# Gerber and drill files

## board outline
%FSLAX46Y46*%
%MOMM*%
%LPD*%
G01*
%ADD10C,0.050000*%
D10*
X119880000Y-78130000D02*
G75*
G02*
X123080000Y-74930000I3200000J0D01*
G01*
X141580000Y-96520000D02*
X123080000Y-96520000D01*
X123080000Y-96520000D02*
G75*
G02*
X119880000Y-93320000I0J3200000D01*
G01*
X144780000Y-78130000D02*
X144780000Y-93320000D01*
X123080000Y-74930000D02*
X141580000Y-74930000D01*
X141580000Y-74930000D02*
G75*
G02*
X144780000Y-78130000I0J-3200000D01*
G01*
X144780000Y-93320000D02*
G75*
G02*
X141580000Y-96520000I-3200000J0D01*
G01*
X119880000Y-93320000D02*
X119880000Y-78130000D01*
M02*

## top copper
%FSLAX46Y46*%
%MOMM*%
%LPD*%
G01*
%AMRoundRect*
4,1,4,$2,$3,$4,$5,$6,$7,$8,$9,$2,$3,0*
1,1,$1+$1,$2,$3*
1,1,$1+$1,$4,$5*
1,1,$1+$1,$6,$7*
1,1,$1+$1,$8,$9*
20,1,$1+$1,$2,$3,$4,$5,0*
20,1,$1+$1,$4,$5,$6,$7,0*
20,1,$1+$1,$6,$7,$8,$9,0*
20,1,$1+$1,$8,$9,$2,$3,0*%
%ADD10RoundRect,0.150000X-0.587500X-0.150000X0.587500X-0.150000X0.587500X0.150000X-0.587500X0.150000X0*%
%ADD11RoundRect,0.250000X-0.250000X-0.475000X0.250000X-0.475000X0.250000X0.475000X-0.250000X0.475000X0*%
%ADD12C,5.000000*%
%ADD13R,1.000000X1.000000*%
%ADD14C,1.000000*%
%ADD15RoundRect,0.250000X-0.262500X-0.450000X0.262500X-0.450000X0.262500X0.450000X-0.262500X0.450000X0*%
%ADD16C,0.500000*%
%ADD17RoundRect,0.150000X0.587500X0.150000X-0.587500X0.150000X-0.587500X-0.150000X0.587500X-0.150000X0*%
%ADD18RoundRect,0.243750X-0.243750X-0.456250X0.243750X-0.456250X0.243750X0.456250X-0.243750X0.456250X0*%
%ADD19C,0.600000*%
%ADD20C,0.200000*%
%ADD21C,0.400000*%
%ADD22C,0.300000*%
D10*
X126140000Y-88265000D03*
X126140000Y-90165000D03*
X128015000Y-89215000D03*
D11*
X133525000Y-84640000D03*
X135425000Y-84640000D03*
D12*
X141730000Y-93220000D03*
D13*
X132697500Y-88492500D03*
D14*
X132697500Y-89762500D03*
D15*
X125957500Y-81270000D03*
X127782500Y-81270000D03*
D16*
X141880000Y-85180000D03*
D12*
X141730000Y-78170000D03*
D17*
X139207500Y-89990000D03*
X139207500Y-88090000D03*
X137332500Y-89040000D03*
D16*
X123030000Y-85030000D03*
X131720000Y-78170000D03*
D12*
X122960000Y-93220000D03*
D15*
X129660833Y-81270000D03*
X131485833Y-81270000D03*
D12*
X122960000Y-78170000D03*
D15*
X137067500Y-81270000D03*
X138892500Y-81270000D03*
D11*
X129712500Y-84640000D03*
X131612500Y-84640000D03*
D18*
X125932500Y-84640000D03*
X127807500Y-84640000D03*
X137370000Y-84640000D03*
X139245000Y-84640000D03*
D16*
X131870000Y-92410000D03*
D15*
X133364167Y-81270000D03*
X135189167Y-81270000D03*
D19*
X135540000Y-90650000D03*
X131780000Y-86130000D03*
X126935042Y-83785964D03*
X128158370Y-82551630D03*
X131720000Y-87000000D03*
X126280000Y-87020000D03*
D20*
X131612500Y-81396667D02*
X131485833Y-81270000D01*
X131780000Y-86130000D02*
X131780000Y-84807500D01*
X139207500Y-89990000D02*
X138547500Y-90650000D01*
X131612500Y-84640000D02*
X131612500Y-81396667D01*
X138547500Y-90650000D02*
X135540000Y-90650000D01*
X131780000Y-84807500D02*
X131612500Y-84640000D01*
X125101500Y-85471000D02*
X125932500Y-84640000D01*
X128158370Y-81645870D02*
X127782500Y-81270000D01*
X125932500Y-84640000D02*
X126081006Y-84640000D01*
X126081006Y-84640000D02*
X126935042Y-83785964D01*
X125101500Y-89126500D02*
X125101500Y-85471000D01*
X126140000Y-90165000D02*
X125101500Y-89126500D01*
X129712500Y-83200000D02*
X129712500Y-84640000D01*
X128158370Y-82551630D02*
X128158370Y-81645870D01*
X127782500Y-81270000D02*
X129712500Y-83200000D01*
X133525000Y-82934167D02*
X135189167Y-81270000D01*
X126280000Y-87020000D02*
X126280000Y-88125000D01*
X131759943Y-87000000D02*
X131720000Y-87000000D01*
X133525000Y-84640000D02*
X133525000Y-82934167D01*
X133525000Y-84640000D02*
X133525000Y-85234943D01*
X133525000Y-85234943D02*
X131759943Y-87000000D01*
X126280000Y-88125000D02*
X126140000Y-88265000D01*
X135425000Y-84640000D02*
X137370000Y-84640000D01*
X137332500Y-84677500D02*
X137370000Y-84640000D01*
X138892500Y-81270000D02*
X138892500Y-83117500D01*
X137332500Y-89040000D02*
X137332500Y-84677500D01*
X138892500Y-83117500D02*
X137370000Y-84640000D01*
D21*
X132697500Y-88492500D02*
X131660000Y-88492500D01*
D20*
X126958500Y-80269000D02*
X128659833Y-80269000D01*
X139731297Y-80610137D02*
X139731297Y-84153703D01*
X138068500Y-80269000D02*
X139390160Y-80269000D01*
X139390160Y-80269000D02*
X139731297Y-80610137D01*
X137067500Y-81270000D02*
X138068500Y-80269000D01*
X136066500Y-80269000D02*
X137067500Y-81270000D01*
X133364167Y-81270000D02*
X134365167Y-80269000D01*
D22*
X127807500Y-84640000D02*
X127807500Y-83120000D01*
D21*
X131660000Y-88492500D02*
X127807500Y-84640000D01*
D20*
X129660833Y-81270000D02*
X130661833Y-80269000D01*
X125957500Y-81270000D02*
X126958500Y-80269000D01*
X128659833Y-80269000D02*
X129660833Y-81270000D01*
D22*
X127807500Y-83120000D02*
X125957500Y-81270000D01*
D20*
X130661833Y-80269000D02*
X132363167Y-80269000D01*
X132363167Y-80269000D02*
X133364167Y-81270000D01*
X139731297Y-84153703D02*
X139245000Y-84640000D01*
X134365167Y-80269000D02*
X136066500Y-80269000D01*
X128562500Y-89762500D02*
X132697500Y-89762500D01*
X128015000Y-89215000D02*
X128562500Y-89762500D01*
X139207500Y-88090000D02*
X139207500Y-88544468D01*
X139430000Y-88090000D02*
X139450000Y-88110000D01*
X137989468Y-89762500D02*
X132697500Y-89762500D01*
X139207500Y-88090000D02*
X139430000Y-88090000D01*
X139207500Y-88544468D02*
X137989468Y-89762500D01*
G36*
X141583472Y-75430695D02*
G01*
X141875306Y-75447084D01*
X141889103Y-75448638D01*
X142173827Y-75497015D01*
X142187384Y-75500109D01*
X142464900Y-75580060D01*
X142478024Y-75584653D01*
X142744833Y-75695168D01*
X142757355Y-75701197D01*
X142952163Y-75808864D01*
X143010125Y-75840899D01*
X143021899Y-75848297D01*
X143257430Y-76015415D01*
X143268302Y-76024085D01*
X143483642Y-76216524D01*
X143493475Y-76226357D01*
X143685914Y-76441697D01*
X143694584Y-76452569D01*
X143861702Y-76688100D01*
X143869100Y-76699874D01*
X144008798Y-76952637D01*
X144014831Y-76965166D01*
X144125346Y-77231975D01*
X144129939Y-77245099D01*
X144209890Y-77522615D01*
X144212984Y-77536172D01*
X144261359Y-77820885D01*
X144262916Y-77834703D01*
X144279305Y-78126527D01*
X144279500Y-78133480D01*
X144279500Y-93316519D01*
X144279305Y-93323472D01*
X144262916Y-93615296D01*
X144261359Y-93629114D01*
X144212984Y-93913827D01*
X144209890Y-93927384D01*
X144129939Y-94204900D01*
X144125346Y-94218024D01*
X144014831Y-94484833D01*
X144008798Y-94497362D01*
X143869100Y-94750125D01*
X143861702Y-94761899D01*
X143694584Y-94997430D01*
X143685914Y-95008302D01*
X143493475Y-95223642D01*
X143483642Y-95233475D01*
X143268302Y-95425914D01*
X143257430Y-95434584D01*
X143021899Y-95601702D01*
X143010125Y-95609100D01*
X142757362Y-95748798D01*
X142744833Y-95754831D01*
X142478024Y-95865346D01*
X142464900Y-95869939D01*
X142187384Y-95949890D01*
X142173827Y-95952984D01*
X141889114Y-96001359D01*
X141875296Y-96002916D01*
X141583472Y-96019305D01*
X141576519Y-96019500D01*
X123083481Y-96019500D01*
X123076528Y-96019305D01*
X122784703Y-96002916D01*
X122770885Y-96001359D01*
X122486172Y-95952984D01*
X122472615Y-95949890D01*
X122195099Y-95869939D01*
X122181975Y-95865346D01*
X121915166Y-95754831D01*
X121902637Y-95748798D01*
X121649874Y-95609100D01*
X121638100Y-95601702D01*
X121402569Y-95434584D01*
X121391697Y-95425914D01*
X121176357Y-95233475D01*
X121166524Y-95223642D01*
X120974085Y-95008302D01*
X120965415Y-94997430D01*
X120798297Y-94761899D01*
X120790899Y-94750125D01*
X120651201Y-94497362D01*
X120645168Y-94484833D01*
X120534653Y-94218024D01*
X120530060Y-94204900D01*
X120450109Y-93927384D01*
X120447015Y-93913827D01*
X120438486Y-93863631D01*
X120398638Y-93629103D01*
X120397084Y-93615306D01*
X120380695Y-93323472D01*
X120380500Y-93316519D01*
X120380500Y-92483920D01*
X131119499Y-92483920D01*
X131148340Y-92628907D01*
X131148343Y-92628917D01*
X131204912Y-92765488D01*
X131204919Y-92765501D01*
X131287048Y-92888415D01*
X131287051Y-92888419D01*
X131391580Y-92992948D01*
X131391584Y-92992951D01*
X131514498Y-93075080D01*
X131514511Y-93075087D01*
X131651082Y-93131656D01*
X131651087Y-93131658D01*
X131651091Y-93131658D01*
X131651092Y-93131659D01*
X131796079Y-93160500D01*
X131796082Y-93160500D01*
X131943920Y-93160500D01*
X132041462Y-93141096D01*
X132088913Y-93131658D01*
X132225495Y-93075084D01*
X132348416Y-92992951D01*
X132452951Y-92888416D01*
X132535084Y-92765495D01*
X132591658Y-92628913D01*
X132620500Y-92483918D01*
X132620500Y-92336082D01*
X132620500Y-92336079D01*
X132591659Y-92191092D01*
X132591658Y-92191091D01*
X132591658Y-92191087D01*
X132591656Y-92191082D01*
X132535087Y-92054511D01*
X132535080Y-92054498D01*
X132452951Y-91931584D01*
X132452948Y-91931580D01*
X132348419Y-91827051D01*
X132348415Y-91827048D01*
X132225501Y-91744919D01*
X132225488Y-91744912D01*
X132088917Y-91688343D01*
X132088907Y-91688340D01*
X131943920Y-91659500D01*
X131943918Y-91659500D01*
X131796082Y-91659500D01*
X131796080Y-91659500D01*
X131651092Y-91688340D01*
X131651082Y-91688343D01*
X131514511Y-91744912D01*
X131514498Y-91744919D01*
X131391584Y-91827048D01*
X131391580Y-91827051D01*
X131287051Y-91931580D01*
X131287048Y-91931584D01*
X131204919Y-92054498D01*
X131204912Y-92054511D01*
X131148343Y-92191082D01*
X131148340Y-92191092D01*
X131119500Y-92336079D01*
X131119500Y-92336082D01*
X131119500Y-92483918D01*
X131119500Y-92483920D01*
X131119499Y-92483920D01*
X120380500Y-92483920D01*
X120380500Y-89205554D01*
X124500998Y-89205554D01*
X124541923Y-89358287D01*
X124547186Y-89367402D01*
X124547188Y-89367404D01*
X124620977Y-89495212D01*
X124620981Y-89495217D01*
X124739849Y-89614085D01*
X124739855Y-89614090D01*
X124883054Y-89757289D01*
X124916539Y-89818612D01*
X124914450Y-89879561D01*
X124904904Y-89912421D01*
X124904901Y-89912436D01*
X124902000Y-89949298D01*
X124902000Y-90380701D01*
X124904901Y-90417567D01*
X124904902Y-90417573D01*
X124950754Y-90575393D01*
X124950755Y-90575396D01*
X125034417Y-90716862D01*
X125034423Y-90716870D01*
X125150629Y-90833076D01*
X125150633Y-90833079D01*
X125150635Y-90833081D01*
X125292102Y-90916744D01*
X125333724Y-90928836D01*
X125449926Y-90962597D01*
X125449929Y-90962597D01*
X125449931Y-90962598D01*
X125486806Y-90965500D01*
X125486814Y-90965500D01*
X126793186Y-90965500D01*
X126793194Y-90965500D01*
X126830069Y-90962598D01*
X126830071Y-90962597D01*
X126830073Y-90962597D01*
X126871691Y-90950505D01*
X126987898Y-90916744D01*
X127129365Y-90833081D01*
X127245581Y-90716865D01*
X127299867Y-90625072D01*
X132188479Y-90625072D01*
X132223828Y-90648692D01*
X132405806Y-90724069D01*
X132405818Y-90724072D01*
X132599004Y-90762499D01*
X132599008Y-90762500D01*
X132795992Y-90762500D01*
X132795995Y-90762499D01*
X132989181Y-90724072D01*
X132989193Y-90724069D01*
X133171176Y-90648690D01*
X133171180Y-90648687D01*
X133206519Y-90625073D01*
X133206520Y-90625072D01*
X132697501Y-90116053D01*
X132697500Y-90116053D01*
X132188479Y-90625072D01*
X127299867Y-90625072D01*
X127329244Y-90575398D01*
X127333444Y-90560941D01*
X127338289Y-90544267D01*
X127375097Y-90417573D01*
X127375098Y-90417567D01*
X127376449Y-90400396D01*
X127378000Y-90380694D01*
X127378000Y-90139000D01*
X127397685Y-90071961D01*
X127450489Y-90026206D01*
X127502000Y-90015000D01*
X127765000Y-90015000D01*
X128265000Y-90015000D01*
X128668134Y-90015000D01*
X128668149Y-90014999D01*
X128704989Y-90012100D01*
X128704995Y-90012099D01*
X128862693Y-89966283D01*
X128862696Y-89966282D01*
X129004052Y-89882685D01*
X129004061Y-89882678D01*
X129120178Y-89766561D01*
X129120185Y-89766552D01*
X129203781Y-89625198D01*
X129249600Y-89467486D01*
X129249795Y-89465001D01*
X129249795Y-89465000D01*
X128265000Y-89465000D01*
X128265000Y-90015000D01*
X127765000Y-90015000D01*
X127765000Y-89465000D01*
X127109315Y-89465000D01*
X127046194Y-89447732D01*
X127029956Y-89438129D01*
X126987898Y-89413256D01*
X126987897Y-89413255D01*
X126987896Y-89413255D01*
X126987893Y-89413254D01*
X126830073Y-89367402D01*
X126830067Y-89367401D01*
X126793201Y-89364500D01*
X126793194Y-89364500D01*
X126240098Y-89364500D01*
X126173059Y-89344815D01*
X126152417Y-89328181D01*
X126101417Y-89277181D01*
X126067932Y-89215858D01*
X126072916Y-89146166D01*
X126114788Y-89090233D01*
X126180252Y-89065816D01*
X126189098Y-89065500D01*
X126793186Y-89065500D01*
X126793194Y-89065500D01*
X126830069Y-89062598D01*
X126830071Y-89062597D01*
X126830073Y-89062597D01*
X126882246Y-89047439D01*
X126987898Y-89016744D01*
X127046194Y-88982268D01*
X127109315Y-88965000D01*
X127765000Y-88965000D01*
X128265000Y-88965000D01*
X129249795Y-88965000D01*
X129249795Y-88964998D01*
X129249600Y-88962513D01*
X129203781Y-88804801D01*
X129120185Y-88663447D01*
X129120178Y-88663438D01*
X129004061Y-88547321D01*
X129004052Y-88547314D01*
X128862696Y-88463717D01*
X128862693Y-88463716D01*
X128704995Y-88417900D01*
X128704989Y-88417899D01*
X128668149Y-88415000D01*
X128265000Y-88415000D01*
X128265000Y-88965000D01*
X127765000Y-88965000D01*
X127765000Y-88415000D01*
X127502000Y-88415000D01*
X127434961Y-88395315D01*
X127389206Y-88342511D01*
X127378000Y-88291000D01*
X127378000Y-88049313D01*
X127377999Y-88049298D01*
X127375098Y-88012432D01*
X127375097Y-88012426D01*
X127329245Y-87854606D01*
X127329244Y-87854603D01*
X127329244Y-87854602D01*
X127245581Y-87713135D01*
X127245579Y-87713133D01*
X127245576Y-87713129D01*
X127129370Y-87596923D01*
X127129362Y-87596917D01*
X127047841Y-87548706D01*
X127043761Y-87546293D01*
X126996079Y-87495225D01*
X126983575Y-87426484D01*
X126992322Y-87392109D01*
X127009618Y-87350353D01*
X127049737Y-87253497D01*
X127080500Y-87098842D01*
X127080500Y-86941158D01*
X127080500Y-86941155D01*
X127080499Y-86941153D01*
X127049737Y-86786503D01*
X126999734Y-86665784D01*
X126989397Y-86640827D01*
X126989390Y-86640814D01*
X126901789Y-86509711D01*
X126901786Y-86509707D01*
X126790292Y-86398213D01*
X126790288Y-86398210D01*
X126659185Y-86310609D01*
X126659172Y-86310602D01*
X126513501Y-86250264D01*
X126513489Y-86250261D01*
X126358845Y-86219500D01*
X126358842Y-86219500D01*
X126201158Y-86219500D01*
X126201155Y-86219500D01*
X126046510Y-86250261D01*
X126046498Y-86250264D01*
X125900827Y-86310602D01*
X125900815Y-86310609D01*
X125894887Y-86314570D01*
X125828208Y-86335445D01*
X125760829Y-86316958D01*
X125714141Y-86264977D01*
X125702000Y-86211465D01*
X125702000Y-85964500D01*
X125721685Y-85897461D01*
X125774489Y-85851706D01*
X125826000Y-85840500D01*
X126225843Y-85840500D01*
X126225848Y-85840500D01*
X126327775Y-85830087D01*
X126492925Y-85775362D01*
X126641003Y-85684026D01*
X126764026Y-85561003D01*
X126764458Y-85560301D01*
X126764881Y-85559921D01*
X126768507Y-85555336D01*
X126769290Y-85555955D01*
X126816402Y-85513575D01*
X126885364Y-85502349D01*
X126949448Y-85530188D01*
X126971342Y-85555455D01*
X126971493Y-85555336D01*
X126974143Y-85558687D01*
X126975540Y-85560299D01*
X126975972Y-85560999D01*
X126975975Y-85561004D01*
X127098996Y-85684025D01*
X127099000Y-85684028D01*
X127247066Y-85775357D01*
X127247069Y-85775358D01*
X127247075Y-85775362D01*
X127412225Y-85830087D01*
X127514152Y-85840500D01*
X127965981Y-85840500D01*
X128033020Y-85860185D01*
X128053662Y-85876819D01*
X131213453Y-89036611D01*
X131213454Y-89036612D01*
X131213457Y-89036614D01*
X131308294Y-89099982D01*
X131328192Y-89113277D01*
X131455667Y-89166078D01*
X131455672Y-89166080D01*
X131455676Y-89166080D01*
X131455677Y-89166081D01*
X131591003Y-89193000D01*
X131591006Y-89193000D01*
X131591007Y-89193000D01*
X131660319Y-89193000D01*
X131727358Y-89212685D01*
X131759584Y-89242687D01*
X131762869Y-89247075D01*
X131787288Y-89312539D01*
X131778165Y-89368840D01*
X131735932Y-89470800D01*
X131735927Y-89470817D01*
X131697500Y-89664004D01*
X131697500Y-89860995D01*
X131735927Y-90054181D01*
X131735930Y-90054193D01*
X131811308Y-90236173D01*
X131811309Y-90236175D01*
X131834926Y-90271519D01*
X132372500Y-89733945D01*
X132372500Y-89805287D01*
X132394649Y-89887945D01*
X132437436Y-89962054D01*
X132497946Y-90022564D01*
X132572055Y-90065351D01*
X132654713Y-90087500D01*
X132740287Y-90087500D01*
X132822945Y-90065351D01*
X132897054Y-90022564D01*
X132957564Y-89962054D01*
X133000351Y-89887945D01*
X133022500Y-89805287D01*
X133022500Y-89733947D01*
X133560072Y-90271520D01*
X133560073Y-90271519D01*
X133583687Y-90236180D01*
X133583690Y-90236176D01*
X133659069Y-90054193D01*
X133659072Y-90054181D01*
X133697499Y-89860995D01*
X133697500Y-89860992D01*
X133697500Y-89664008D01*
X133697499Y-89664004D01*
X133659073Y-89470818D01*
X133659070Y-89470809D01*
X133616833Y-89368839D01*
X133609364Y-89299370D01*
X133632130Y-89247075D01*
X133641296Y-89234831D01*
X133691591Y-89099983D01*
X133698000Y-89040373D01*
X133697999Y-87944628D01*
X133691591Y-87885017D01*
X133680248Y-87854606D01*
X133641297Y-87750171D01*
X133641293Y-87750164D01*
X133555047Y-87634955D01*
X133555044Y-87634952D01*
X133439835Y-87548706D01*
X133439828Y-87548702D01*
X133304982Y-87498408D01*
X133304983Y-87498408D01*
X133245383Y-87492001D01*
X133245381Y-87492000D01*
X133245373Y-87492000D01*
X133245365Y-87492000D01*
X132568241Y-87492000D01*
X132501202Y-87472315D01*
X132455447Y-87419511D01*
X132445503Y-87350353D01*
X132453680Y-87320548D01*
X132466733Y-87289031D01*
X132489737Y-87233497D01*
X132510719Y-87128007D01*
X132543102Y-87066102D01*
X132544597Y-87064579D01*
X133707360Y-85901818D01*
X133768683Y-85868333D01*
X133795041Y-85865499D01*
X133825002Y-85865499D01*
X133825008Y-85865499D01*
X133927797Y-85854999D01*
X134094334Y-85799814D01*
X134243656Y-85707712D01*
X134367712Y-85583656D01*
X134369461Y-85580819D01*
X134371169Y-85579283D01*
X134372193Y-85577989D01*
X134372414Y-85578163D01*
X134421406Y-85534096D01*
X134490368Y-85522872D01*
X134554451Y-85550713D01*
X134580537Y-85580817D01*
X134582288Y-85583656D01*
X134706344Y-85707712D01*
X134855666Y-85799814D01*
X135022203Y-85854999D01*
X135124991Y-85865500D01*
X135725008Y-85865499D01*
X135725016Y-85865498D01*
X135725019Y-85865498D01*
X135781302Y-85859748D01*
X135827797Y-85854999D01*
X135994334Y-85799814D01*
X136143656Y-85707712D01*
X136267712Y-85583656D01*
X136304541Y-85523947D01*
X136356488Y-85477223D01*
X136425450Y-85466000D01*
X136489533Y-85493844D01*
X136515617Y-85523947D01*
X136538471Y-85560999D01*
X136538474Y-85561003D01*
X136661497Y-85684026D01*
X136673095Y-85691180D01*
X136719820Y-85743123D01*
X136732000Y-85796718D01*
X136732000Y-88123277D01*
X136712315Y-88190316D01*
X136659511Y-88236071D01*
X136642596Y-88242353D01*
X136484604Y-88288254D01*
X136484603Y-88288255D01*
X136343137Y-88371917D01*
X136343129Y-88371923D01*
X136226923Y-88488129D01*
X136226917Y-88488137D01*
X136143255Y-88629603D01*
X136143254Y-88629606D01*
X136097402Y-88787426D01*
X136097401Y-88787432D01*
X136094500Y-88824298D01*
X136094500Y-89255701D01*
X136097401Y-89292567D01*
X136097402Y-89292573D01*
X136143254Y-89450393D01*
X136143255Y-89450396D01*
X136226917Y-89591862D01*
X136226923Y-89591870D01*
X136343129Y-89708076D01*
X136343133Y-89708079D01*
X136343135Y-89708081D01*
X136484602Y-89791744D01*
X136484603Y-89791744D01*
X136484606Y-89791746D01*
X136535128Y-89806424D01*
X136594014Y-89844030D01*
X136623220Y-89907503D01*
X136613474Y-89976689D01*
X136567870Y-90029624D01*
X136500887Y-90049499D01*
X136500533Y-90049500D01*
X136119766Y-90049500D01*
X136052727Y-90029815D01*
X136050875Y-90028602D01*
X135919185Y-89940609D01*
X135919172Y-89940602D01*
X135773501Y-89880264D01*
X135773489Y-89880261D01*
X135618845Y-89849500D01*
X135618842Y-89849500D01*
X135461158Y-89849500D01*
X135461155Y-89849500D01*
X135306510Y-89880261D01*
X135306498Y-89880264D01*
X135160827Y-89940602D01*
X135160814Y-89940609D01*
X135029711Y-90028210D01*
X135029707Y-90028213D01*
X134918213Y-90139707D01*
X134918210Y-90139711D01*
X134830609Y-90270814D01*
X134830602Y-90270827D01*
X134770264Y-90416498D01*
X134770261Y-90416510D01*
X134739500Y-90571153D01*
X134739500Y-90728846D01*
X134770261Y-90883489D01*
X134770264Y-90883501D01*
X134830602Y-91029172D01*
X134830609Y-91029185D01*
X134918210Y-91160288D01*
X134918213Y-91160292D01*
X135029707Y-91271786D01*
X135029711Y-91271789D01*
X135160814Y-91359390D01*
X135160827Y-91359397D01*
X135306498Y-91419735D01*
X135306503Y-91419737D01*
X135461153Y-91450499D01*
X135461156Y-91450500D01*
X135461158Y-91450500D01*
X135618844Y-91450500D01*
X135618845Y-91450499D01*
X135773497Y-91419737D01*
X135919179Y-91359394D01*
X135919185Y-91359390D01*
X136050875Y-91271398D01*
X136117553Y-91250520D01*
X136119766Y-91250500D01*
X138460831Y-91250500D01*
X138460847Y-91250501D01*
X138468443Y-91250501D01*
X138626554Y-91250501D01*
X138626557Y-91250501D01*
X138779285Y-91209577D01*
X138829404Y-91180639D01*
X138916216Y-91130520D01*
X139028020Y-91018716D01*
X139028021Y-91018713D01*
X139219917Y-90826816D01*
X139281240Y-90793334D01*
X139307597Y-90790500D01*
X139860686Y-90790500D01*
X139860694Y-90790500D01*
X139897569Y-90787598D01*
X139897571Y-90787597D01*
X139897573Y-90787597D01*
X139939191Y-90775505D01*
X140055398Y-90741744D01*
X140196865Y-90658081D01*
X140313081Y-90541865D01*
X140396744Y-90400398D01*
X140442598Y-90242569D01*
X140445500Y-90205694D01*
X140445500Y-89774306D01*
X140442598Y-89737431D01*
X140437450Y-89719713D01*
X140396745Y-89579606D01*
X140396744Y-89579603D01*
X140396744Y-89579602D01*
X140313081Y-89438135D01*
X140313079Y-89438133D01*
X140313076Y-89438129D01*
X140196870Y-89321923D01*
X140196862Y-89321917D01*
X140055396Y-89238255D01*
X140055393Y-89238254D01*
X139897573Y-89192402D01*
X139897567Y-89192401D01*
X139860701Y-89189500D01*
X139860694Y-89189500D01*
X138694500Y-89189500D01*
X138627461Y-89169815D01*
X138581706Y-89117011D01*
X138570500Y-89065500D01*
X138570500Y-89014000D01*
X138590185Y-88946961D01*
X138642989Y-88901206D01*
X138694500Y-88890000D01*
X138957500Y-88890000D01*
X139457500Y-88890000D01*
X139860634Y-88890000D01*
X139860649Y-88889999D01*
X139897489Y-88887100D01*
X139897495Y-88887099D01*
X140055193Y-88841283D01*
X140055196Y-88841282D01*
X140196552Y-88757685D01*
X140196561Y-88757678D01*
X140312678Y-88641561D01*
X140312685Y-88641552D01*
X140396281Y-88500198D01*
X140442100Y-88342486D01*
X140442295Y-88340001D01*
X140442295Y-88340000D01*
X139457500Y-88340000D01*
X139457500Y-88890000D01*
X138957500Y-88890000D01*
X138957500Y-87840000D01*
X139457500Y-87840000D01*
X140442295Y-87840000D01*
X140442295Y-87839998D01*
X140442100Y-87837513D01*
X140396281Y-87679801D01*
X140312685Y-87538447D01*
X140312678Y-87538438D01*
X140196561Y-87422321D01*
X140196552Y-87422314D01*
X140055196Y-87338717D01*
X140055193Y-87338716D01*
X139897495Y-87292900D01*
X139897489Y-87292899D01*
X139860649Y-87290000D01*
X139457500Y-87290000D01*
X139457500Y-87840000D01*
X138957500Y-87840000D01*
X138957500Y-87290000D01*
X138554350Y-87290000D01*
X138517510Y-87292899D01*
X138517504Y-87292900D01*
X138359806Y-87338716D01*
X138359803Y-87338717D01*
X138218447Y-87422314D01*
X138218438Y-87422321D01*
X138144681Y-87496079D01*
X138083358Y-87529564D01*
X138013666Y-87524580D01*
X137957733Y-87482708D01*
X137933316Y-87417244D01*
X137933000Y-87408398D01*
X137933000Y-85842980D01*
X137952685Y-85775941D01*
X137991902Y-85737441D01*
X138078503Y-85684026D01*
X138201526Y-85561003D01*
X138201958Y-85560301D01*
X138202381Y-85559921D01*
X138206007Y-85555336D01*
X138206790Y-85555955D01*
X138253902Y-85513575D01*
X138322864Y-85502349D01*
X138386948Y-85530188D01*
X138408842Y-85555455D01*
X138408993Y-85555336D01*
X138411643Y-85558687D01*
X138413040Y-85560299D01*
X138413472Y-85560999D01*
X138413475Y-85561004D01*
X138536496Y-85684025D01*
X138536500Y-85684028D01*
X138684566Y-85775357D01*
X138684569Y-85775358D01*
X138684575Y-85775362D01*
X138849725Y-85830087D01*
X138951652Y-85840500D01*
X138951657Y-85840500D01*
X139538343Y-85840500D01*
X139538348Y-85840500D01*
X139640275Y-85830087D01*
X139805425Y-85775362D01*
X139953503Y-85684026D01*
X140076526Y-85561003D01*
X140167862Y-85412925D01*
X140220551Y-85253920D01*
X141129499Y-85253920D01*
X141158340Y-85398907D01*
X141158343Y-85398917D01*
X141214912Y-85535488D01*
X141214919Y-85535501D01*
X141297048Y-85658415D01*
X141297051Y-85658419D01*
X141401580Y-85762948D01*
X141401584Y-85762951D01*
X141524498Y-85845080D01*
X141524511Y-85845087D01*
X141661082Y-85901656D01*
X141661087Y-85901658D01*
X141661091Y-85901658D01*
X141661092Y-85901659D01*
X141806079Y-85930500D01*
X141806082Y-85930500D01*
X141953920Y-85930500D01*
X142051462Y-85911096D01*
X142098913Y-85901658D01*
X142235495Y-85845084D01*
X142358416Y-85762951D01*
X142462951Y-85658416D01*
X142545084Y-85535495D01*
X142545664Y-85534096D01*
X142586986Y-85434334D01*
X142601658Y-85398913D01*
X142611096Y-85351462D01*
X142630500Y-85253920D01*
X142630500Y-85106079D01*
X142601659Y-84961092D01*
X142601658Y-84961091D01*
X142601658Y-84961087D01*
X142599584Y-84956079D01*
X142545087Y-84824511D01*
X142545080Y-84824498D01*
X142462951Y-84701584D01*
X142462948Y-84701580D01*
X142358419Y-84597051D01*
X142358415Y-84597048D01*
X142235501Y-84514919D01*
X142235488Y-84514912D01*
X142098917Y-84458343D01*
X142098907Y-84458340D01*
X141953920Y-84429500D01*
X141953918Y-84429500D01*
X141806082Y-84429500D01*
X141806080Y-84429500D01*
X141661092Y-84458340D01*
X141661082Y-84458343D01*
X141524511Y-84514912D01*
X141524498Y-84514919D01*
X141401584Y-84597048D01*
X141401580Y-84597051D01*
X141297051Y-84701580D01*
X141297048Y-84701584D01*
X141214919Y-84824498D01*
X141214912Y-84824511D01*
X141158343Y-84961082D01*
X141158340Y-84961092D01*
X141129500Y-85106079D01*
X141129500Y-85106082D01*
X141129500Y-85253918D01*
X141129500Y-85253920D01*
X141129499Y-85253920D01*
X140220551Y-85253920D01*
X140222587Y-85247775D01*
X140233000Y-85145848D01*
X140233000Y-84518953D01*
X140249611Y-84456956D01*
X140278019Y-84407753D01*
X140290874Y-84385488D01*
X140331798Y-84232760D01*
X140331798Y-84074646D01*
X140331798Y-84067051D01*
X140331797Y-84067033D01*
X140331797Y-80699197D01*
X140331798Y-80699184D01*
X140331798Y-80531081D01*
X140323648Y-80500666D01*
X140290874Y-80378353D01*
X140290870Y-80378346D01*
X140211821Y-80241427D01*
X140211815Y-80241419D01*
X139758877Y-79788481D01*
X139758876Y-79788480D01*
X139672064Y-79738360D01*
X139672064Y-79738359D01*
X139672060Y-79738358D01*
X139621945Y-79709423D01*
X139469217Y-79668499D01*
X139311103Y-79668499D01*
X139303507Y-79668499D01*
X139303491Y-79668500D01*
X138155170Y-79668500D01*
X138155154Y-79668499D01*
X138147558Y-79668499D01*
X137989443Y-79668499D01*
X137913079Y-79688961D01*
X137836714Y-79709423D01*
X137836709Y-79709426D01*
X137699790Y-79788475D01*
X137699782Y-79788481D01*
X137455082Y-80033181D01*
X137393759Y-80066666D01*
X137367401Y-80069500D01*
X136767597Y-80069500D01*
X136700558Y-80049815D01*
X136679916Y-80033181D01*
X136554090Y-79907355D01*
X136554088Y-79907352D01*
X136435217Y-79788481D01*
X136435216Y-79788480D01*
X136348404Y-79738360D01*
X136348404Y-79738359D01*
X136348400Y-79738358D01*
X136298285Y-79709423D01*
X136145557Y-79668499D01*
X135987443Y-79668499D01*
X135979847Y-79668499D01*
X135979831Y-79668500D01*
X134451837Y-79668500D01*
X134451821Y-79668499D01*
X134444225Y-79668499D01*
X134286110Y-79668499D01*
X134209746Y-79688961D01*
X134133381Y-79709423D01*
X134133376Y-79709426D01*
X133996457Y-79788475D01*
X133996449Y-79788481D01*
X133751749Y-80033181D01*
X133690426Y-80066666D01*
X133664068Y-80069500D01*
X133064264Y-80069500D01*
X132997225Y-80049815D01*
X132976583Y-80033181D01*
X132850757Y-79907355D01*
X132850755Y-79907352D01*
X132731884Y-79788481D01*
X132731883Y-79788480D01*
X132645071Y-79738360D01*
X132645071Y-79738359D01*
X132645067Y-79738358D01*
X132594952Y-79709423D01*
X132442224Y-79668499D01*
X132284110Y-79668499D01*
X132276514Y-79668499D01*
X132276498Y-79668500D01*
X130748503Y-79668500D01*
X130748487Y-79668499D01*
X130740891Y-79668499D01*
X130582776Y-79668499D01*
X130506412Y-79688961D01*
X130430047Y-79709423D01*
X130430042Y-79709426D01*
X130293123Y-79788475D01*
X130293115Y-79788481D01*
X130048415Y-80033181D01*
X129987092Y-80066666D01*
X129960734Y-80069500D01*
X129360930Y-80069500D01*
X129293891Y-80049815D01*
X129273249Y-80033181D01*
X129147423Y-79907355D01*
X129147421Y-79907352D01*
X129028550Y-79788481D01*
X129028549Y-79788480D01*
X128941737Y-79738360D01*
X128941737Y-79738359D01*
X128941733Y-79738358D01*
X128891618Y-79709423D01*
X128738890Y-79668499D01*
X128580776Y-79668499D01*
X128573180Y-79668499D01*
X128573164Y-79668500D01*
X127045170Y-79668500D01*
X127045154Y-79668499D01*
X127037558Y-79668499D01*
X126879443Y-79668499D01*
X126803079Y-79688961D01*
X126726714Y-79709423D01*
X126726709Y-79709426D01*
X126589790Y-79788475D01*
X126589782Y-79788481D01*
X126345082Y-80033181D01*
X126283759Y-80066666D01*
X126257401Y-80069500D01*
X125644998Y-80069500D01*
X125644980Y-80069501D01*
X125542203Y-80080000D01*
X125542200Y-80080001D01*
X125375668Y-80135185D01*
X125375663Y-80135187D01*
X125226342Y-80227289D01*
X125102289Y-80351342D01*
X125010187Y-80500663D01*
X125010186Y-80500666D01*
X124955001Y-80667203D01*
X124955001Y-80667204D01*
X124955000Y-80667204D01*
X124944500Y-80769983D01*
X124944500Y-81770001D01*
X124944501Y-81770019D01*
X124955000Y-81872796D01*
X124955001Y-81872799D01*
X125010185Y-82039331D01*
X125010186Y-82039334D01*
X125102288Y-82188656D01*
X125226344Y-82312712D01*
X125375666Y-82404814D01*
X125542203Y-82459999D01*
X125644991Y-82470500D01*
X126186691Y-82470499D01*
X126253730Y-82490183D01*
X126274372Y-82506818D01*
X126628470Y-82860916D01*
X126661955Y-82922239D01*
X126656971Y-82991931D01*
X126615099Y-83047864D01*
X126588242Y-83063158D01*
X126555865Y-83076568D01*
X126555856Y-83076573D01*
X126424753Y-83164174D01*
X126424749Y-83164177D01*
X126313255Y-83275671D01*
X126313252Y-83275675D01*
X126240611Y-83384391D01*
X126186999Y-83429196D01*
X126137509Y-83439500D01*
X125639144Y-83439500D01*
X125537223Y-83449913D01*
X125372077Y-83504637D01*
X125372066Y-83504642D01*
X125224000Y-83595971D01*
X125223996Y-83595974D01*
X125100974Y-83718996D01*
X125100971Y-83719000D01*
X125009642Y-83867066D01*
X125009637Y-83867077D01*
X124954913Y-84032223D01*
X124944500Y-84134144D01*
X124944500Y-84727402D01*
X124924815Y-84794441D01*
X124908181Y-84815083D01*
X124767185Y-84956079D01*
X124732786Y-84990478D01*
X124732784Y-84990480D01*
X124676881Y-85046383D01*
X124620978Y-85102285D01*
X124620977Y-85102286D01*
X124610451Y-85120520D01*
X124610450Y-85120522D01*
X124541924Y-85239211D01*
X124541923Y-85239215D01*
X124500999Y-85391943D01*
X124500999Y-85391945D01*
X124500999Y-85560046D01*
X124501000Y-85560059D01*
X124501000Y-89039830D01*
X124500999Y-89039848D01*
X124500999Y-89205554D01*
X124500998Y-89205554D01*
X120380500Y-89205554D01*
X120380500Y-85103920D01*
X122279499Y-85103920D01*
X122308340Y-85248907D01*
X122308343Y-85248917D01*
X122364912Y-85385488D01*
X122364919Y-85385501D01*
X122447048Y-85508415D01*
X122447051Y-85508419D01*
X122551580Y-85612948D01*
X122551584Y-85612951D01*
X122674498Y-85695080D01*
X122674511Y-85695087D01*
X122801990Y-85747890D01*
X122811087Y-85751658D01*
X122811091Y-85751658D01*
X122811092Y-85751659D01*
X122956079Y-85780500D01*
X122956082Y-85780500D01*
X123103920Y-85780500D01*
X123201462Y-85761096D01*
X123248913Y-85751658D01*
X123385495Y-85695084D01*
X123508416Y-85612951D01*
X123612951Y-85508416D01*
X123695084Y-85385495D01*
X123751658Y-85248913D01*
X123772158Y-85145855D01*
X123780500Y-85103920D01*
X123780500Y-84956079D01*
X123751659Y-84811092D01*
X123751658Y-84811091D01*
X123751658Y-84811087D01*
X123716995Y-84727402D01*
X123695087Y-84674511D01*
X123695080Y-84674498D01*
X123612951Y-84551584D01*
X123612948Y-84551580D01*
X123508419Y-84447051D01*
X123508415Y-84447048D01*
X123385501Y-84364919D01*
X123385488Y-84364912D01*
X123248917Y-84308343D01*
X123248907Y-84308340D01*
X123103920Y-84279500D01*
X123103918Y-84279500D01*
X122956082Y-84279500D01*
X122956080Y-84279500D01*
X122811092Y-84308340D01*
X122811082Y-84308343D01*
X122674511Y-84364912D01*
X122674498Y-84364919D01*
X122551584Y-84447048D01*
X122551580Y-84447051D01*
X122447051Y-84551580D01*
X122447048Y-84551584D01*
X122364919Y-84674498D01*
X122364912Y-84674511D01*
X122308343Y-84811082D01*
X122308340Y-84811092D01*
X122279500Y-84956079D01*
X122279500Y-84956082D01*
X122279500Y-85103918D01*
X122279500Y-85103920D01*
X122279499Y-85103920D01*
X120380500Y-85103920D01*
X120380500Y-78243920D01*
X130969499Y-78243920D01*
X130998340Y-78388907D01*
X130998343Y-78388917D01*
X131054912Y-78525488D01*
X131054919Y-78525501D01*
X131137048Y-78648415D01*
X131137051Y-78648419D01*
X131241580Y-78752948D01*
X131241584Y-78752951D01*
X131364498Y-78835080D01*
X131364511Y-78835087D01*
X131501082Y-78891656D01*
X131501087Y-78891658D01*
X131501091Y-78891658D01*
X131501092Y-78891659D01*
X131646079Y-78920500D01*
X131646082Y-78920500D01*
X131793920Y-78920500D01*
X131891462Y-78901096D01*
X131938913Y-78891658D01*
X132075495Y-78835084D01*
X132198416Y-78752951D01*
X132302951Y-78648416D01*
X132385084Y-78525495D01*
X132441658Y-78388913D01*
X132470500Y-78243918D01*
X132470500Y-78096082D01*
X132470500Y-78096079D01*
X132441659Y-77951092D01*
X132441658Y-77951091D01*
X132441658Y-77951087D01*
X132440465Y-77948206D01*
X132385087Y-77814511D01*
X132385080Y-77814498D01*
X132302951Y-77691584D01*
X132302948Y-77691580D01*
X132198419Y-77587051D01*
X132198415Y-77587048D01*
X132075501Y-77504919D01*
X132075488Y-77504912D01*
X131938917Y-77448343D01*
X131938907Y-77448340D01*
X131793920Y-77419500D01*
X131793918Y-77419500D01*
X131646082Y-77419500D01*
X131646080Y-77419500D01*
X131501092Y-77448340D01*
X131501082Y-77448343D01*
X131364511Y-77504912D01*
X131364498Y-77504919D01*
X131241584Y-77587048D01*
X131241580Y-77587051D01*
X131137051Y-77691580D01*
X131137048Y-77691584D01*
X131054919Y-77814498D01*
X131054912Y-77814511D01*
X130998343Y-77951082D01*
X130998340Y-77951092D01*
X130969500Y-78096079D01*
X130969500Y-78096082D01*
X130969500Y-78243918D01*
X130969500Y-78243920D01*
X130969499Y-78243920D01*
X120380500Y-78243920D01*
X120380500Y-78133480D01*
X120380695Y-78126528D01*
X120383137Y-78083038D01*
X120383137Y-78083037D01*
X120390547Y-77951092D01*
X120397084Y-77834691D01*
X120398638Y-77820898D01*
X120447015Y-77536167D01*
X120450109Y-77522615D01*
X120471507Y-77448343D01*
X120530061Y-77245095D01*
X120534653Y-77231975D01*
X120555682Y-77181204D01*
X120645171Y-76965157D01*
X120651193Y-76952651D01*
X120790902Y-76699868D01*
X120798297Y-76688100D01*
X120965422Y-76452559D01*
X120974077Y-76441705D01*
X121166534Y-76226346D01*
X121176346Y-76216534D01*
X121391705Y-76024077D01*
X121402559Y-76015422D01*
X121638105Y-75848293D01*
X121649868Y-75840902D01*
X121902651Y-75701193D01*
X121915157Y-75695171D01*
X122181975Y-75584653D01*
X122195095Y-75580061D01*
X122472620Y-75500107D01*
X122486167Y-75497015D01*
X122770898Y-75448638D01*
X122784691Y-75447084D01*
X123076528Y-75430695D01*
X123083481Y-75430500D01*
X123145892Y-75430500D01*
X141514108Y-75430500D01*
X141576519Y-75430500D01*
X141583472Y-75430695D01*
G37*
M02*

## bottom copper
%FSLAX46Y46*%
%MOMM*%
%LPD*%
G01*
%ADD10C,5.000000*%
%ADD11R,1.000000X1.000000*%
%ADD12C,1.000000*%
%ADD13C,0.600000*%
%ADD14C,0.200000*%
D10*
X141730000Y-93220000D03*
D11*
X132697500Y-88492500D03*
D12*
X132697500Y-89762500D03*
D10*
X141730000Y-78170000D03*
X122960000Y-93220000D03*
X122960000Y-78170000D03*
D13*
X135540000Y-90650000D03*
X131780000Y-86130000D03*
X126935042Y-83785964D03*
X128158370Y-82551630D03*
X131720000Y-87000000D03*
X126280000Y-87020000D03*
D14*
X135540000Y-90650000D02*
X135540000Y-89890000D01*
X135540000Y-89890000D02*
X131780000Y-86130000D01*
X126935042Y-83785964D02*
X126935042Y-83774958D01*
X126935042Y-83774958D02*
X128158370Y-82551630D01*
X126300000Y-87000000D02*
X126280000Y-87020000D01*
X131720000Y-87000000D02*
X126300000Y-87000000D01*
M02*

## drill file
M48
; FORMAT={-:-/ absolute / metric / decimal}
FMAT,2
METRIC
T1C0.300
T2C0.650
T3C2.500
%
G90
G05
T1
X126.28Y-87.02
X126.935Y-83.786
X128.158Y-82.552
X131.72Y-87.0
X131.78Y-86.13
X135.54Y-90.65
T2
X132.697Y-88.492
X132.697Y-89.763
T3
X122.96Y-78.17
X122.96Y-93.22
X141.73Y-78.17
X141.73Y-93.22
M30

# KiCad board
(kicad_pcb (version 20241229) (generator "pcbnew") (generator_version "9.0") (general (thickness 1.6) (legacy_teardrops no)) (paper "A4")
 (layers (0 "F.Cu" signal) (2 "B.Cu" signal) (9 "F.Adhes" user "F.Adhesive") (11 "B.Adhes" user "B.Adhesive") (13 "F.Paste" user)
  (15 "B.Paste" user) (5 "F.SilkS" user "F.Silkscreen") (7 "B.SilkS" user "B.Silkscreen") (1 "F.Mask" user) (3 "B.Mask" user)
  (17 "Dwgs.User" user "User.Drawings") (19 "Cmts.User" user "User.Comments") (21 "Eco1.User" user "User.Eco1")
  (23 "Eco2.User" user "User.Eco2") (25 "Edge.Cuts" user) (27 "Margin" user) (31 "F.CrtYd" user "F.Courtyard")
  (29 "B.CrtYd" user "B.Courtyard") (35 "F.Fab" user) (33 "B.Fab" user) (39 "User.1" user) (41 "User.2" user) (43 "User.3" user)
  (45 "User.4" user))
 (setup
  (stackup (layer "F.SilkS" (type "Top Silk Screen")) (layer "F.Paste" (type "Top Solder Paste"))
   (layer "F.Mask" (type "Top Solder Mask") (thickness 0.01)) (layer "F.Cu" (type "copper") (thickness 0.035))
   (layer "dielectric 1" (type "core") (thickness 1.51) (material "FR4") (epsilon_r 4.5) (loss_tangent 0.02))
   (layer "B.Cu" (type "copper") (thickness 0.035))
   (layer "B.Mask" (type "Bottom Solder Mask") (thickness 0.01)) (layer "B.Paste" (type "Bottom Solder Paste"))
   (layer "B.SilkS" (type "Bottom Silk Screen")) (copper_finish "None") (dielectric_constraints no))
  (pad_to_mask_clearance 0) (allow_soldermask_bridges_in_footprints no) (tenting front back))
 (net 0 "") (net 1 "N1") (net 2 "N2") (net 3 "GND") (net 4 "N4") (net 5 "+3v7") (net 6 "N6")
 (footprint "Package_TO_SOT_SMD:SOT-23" (layer "F.Cu") (at 127.0775 89.215)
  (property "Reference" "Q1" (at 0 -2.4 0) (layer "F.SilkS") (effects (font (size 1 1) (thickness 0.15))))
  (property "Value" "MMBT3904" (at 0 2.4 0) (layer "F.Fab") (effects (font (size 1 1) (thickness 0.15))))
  (pad "1" smd roundrect (at -0.9375 -0.95) (size 1.475 0.6) (layers "F.Cu" "F.Mask" "F.Paste") (roundrect_rratio 0.25) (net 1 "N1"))
  (pad "2" smd roundrect (at -0.9375 0.95) (size 1.475 0.6) (layers "F.Cu" "F.Mask" "F.Paste") (roundrect_rratio 0.25) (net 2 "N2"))
  (pad "3" smd roundrect (at 0.9375 0) (size 1.475 0.6) (layers "F.Cu" "F.Mask" "F.Paste") (roundrect_rratio 0.25) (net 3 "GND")))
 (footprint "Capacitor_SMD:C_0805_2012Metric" (layer "F.Cu") (at 134.475 84.64)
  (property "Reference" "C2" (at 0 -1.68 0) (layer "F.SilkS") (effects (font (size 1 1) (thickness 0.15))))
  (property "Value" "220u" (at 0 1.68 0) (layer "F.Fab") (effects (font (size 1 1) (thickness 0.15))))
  (pad "1" smd roundrect (at -0.95 0) (size 1 1.45) (layers "F.Cu" "F.Mask" "F.Paste") (roundrect_rratio 0.25) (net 1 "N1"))
  (pad "2" smd roundrect (at 0.95 0) (size 1 1.45) (layers "F.Cu" "F.Mask" "F.Paste") (roundrect_rratio 0.25) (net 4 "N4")))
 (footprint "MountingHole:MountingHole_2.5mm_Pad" (layer "F.Cu") (at 141.73 93.22)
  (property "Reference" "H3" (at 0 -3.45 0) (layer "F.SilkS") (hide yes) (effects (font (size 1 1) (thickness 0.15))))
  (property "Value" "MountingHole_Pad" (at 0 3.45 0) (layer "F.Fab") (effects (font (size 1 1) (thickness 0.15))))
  (pad "1" thru_hole circle (at 0 0) (size 5 5) (drill 2.5) (layers "*.Cu" "*.Mask") (remove_unused_layers no) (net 3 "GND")
   (zone_connect 2)))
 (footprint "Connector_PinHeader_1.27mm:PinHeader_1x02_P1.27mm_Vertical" (layer "F.Cu") (at 132.6975 88.4925)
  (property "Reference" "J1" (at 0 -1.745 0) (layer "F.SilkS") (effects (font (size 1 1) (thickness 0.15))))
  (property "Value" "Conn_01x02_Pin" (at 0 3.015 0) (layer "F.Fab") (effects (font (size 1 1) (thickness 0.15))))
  (pad "1" thru_hole rect (at 0 0) (size 1 1) (drill 0.65) (layers "*.Cu" "*.Mask") (remove_unused_layers no) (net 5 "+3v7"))
  (pad "2" thru_hole circle (at 0 1.27) (size 1 1) (drill 0.65) (layers "*.Cu" "*.Mask") (remove_unused_layers no) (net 3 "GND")))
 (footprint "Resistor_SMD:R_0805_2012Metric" (layer "F.Cu") (at 126.87 81.27)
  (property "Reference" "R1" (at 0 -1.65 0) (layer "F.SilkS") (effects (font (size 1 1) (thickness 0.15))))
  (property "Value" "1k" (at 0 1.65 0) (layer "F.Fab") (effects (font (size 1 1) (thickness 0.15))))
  (pad "1" smd roundrect (at -0.9125 0) (size 1.025 1.4) (layers "F.Cu" "F.Mask" "F.Paste") (roundrect_rratio 0.243902) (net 5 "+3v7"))
  (pad "2" smd roundrect (at 0.9125 0) (size 1.025 1.4) (layers "F.Cu" "F.Mask" "F.Paste") (roundrect_rratio 0.243902) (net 2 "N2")))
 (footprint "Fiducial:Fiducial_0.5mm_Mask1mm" (layer "F.Cu") (at 141.88 85.18)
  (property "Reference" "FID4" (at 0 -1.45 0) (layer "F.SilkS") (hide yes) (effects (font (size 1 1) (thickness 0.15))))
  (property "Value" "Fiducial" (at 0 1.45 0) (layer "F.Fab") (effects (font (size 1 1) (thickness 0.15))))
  (pad "" smd circle (at 0 0) (size 0.5 0.5) (layers "F.Cu" "F.Mask") (solder_mask_margin 0.25)))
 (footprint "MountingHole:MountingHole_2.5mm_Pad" (layer "F.Cu") (at 141.73 78.17)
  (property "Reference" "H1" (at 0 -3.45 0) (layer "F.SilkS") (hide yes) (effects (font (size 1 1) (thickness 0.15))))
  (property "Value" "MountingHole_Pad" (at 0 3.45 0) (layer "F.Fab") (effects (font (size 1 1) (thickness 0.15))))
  (pad "1" thru_hole circle (at 0 0) (size 5 5) (drill 2.5) (layers "*.Cu" "*.Mask") (remove_unused_layers no) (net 3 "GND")
   (zone_connect 2)))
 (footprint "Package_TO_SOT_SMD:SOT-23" (layer "F.Cu") (at 138.27 89.04 180)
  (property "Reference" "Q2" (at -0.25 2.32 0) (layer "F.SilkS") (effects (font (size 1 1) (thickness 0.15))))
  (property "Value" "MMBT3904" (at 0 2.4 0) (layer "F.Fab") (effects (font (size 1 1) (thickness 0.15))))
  (pad "1" smd roundrect (at -0.9375 -0.95 180) (size 1.475 0.6) (layers "F.Cu" "F.Mask" "F.Paste") (roundrect_rratio 0.25) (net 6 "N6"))
  (pad "2" smd roundrect (at -0.9375 0.95 180) (size 1.475 0.6) (layers "F.Cu" "F.Mask" "F.Paste") (roundrect_rratio 0.25) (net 3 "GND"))
  (pad "3" smd roundrect (at 0.9375 0 180) (size 1.475 0.6) (layers "F.Cu" "F.Mask" "F.Paste") (roundrect_rratio 0.25) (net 4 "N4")))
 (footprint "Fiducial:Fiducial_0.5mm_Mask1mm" (layer "F.Cu") (at 123.03 85.03)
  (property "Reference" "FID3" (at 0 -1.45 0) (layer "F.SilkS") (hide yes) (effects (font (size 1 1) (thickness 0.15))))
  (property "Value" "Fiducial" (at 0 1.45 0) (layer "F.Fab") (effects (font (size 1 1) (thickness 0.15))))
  (pad "" smd circle (at 0 0) (size 0.5 0.5) (layers "F.Cu" "F.Mask") (solder_mask_margin 0.25)))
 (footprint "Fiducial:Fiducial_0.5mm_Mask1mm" (layer "F.Cu") (at 131.72 78.17)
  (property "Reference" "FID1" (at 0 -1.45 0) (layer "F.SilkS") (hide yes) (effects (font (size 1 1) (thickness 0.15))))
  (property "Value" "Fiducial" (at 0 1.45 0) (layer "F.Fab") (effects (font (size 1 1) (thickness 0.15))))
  (pad "" smd circle (at 0 0) (size 0.5 0.5) (layers "F.Cu" "F.Mask") (solder_mask_margin 0.25)))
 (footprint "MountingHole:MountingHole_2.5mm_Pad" (layer "F.Cu") (at 122.96 93.22)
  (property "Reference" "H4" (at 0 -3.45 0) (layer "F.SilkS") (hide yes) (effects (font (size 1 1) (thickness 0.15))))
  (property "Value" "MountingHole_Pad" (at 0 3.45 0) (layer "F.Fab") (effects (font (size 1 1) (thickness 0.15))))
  (pad "1" thru_hole circle (at 0 0) (size 5 5) (drill 2.5) (layers "*.Cu" "*.Mask") (remove_unused_layers no) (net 3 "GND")
   (zone_connect 2)))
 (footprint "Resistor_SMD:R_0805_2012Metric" (layer "F.Cu") (at 130.573333 81.27)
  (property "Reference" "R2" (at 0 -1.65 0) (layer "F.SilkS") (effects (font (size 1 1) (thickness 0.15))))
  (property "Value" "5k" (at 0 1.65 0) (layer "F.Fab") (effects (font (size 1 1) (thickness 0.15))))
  (pad "1" smd roundrect (at -0.9125 0) (size 1.025 1.4) (layers "F.Cu" "F.Mask" "F.Paste") (roundrect_rratio 0.243902) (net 5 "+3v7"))
  (pad "2" smd roundrect (at 0.9125 0) (size 1.025 1.4) (layers "F.Cu" "F.Mask" "F.Paste") (roundrect_rratio 0.243902) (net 6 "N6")))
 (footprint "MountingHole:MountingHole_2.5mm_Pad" (layer "F.Cu") (at 122.96 78.17)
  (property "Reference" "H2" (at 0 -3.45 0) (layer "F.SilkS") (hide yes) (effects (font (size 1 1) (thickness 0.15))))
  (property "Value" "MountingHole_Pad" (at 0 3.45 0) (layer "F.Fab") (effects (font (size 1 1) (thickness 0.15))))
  (pad "1" thru_hole circle (at 0 0) (size 5 5) (drill 2.5) (layers "*.Cu" "*.Mask") (remove_unused_layers no) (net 3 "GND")
   (zone_connect 2)))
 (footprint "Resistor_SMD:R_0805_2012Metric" (layer "F.Cu") (at 137.98 81.27)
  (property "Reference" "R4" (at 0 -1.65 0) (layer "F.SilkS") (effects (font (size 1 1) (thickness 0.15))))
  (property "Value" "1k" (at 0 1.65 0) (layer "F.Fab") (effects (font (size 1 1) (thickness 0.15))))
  (pad "1" smd roundrect (at -0.9125 0) (size 1.025 1.4) (layers "F.Cu" "F.Mask" "F.Paste") (roundrect_rratio 0.243902) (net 5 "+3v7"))
  (pad "2" smd roundrect (at 0.9125 0) (size 1.025 1.4) (layers "F.Cu" "F.Mask" "F.Paste") (roundrect_rratio 0.243902) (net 4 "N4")))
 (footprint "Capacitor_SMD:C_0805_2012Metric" (layer "F.Cu") (at 130.6625 84.64)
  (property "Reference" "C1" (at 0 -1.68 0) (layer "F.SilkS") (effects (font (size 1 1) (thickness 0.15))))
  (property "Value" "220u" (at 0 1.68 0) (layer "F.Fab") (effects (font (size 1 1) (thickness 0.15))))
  (pad "1" smd roundrect (at -0.95 0) (size 1 1.45) (layers "F.Cu" "F.Mask" "F.Paste") (roundrect_rratio 0.25) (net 2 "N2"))
  (pad "2" smd roundrect (at 0.95 0) (size 1 1.45) (layers "F.Cu" "F.Mask" "F.Paste") (roundrect_rratio 0.25) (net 6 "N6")))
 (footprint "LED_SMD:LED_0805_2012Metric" (layer "F.Cu") (at 126.87 84.64)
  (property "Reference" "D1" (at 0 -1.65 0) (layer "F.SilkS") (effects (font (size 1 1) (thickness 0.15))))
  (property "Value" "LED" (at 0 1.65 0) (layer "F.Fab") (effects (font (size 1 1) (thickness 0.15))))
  (pad "1" smd roundrect (at -0.9375 0) (size 0.975 1.4) (layers "F.Cu" "F.Mask" "F.Paste") (roundrect_rratio 0.25) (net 2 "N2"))
  (pad "2" smd roundrect (at 0.9375 0) (size 0.975 1.4) (layers "F.Cu" "F.Mask" "F.Paste") (roundrect_rratio 0.25) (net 5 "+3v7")))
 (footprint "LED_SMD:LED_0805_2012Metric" (layer "F.Cu") (at 138.3075 84.64)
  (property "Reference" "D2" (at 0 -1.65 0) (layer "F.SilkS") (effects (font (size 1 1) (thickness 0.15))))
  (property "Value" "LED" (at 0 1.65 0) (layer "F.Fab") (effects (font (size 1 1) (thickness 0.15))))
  (pad "1" smd roundrect (at -0.9375 0) (size 0.975 1.4) (layers "F.Cu" "F.Mask" "F.Paste") (roundrect_rratio 0.25) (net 4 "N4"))
  (pad "2" smd roundrect (at 0.9375 0) (size 0.975 1.4) (layers "F.Cu" "F.Mask" "F.Paste") (roundrect_rratio 0.25) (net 5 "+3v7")))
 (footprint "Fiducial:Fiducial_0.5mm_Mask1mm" (layer "F.Cu") (at 131.87 92.41)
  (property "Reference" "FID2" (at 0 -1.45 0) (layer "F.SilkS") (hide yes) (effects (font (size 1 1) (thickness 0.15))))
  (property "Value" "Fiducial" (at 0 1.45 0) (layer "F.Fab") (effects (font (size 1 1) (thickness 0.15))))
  (pad "" smd circle (at 0 0) (size 0.5 0.5) (layers "F.Cu" "F.Mask") (solder_mask_margin 0.25)))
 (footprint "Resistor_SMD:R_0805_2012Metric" (layer "F.Cu") (at 134.276667 81.27)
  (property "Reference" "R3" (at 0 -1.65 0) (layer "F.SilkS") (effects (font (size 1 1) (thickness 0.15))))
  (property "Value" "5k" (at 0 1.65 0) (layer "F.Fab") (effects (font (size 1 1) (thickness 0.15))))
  (pad "1" smd roundrect (at -0.9125 0) (size 1.025 1.4) (layers "F.Cu" "F.Mask" "F.Paste") (roundrect_rratio 0.243902) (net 5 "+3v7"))
  (pad "2" smd roundrect (at 0.9125 0) (size 1.025 1.4) (layers "F.Cu" "F.Mask" "F.Paste") (roundrect_rratio 0.243902) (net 1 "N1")))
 (gr_arc (start 119.88 78.13) (mid 120.817258 75.867258) (end 123.08 74.93) (stroke (width 0.05) (type default)) (layer "Edge.Cuts"))
 (gr_line (start 141.58 96.52) (end 123.08 96.52) (stroke (width 0.05) (type default)) (layer "Edge.Cuts"))
 (gr_arc (start 123.08 96.52) (mid 120.817258 95.582742) (end 119.88 93.32) (stroke (width 0.05) (type default)) (layer "Edge.Cuts"))
 (gr_line (start 144.78 78.13) (end 144.78 93.32) (stroke (width 0.05) (type default)) (layer "Edge.Cuts"))
 (gr_line (start 123.08 74.93) (end 141.58 74.93) (stroke (width 0.05) (type default)) (layer "Edge.Cuts"))
 (gr_arc (start 141.58 74.93) (mid 143.842742 75.867258) (end 144.78 78.13) (stroke (width 0.05) (type default)) (layer "Edge.Cuts"))
 (gr_arc (start 144.78 93.32) (mid 143.842742 95.582742) (end 141.58 96.52) (stroke (width 0.05) (type default)) (layer "Edge.Cuts"))
 (gr_line (start 119.88 93.32) (end 119.88 78.13) (stroke (width 0.05) (type default)) (layer "Edge.Cuts"))
 (segment (start 131.6125 81.396667) (end 131.485833 81.27) (width 0.2) (layer "F.Cu") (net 6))
 (segment (start 131.78 86.13) (end 131.78 84.8075) (width 0.2) (layer "F.Cu") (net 6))
 (segment (start 139.2075 89.99) (end 138.5475 90.65) (width 0.2) (layer "F.Cu") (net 6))
 (segment (start 131.6125 84.64) (end 131.6125 81.396667) (width 0.2) (layer "F.Cu") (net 6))
 (segment (start 138.5475 90.65) (end 135.54 90.65) (width 0.2) (layer "F.Cu") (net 6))
 (segment (start 131.78 84.8075) (end 131.6125 84.64) (width 0.2) (layer "F.Cu") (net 6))
 (via (at 135.54 90.65) (size 0.6) (drill 0.3) (layers "F.Cu" "B.Cu") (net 6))
 (via (at 131.78 86.13) (size 0.6) (drill 0.3) (layers "F.Cu" "B.Cu") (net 6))
 (segment (start 135.54 90.65) (end 135.54 89.89) (width 0.2) (layer "B.Cu") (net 6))
 (segment (start 135.54 89.89) (end 131.78 86.13) (width 0.2) (layer "B.Cu") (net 6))
 (segment (start 125.1015 85.471) (end 125.9325 84.64) (width 0.2) (layer "F.Cu") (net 2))
 (segment (start 128.15837 81.64587) (end 127.7825 81.27) (width 0.2) (layer "F.Cu") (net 2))
 (segment (start 125.9325 84.64) (end 126.081006 84.64) (width 0.2) (layer "F.Cu") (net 2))
 (segment (start 126.081006 84.64) (end 126.935042 83.785964) (width 0.2) (layer "F.Cu") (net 2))
 (segment (start 125.1015 89.1265) (end 125.1015 85.471) (width 0.2) (layer "F.Cu") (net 2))
 (segment (start 126.14 90.165) (end 125.1015 89.1265) (width 0.2) (layer "F.Cu") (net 2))
 (segment (start 129.7125 83.2) (end 129.7125 84.64) (width 0.2) (layer "F.Cu") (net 2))
 (segment (start 128.15837 82.55163) (end 128.15837 81.64587) (width 0.2) (layer "F.Cu") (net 2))
 (segment (start 127.7825 81.27) (end 129.7125 83.2) (width 0.2) (layer "F.Cu") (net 2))
 (via (at 126.935042 83.785964) (size 0.6) (drill 0.3) (layers "F.Cu" "B.Cu") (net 2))
 (via (at 128.15837 82.55163) (size 0.6) (drill 0.3) (layers "F.Cu" "B.Cu") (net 2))
 (segment (start 126.935042 83.785964) (end 126.935042 83.774958) (width 0.2) (layer "B.Cu") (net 2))
 (segment (start 126.935042 83.774958) (end 128.15837 82.55163) (width 0.2) (layer "B.Cu") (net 2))
 (segment (start 133.525 82.934167) (end 135.189167 81.27) (width 0.2) (layer "F.Cu") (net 1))
 (segment (start 126.28 87.02) (end 126.28 88.125) (width 0.2) (layer "F.Cu") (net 1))
 (segment (start 131.759943 87) (end 131.72 87) (width 0.2) (layer "F.Cu") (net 1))
 (segment (start 133.525 84.64) (end 133.525 82.934167) (width 0.2) (layer "F.Cu") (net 1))
 (segment (start 133.525 84.64) (end 133.525 85.234943) (width 0.2) (layer "F.Cu") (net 1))
 (segment (start 133.525 85.234943) (end 131.759943 87) (width 0.2) (layer "F.Cu") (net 1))
 (segment (start 126.28 88.125) (end 126.14 88.265) (width 0.2) (layer "F.Cu") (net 1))
 (via (at 131.72 87) (size 0.6) (drill 0.3) (layers "F.Cu" "B.Cu") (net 1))
 (via (at 126.28 87.02) (size 0.6) (drill 0.3) (layers "F.Cu" "B.Cu") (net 1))
 (segment (start 126.3 87) (end 126.28 87.02) (width 0.2) (layer "B.Cu") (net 1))
 (segment (start 131.72 87) (end 126.3 87) (width 0.2) (layer "B.Cu") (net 1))
 (segment (start 135.425 84.64) (end 137.37 84.64) (width 0.2) (layer "F.Cu") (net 4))
 (segment (start 137.3325 84.6775) (end 137.37 84.64) (width 0.2) (layer "F.Cu") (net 4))
 (segment (start 138.8925 81.27) (end 138.8925 83.1175) (width 0.2) (layer "F.Cu") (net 4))
 (segment (start 137.3325 89.04) (end 137.3325 84.6775) (width 0.2) (layer "F.Cu") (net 4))
 (segment (start 138.8925 83.1175) (end 137.37 84.64) (width 0.2) (layer "F.Cu") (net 4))
 (segment (start 132.6975 88.4925) (end 131.66 88.4925) (width 0.4) (layer "F.Cu") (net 5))
 (segment (start 126.9585 80.269) (end 128.659833 80.269) (width 0.2) (layer "F.Cu") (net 5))
 (segment (start 139.731297 80.610137) (end 139.731297 84.153703) (width 0.2) (layer "F.Cu") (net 5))
 (segment (start 138.0685 80.269) (end 139.39016 80.269) (width 0.2) (layer "F.Cu") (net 5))
 (segment (start 139.39016 80.269) (end 139.731297 80.610137) (width 0.2) (layer "F.Cu") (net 5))
 (segment (start 137.0675 81.27) (end 138.0685 80.269) (width 0.2) (layer "F.Cu") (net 5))
 (segment (start 136.0665 80.269) (end 137.0675 81.27) (width 0.2) (layer "F.Cu") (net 5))
 (segment (start 133.364167 81.27) (end 134.365167 80.269) (width 0.2) (layer "F.Cu") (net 5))
 (segment (start 127.8075 84.64) (end 127.8075 83.12) (width 0.3) (layer "F.Cu") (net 5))
 (segment (start 131.66 88.4925) (end 127.8075 84.64) (width 0.4) (layer "F.Cu") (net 5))
 (segment (start 129.660833 81.27) (end 130.661833 80.269) (width 0.2) (layer "F.Cu") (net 5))
 (segment (start 125.9575 81.27) (end 126.9585 80.269) (width 0.2) (layer "F.Cu") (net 5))
 (segment (start 128.659833 80.269) (end 129.660833 81.27) (width 0.2) (layer "F.Cu") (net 5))
 (segment (start 127.8075 83.12) (end 125.9575 81.27) (width 0.3) (layer "F.Cu") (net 5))
 (segment (start 130.661833 80.269) (end 132.363167 80.269) (width 0.2) (layer "F.Cu") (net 5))
 (segment (start 132.363167 80.269) (end 133.364167 81.27) (width 0.2) (layer "F.Cu") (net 5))
 (segment (start 139.731297 84.153703) (end 139.245 84.64) (width 0.2) (layer "F.Cu") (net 5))
 (segment (start 134.365167 80.269) (end 136.0665 80.269) (width 0.2) (layer "F.Cu") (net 5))
 (segment (start 128.5625 89.7625) (end 132.6975 89.7625) (width 0.2) (layer "F.Cu") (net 3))
 (segment (start 128.015 89.215) (end 128.5625 89.7625) (width 0.2) (layer "F.Cu") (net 3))
 (segment (start 139.2075 88.09) (end 139.2075 88.544468) (width 0.2) (layer "F.Cu") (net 3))
 (segment (start 139.43 88.09) (end 139.45 88.11) (width 0.2) (layer "F.Cu") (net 3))
 (segment (start 137.989468 89.7625) (end 132.6975 89.7625) (width 0.2) (layer "F.Cu") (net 3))
 (segment (start 139.2075 88.09) (end 139.43 88.09) (width 0.2) (layer "F.Cu") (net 3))
 (segment (start 139.2075 88.544468) (end 137.989468 89.7625) (width 0.2) (layer "F.Cu") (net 3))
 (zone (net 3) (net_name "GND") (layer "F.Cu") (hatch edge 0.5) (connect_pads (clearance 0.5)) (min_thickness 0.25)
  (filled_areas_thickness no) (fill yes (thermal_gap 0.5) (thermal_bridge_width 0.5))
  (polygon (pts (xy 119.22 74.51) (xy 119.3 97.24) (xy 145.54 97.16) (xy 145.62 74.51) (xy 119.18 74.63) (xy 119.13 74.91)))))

